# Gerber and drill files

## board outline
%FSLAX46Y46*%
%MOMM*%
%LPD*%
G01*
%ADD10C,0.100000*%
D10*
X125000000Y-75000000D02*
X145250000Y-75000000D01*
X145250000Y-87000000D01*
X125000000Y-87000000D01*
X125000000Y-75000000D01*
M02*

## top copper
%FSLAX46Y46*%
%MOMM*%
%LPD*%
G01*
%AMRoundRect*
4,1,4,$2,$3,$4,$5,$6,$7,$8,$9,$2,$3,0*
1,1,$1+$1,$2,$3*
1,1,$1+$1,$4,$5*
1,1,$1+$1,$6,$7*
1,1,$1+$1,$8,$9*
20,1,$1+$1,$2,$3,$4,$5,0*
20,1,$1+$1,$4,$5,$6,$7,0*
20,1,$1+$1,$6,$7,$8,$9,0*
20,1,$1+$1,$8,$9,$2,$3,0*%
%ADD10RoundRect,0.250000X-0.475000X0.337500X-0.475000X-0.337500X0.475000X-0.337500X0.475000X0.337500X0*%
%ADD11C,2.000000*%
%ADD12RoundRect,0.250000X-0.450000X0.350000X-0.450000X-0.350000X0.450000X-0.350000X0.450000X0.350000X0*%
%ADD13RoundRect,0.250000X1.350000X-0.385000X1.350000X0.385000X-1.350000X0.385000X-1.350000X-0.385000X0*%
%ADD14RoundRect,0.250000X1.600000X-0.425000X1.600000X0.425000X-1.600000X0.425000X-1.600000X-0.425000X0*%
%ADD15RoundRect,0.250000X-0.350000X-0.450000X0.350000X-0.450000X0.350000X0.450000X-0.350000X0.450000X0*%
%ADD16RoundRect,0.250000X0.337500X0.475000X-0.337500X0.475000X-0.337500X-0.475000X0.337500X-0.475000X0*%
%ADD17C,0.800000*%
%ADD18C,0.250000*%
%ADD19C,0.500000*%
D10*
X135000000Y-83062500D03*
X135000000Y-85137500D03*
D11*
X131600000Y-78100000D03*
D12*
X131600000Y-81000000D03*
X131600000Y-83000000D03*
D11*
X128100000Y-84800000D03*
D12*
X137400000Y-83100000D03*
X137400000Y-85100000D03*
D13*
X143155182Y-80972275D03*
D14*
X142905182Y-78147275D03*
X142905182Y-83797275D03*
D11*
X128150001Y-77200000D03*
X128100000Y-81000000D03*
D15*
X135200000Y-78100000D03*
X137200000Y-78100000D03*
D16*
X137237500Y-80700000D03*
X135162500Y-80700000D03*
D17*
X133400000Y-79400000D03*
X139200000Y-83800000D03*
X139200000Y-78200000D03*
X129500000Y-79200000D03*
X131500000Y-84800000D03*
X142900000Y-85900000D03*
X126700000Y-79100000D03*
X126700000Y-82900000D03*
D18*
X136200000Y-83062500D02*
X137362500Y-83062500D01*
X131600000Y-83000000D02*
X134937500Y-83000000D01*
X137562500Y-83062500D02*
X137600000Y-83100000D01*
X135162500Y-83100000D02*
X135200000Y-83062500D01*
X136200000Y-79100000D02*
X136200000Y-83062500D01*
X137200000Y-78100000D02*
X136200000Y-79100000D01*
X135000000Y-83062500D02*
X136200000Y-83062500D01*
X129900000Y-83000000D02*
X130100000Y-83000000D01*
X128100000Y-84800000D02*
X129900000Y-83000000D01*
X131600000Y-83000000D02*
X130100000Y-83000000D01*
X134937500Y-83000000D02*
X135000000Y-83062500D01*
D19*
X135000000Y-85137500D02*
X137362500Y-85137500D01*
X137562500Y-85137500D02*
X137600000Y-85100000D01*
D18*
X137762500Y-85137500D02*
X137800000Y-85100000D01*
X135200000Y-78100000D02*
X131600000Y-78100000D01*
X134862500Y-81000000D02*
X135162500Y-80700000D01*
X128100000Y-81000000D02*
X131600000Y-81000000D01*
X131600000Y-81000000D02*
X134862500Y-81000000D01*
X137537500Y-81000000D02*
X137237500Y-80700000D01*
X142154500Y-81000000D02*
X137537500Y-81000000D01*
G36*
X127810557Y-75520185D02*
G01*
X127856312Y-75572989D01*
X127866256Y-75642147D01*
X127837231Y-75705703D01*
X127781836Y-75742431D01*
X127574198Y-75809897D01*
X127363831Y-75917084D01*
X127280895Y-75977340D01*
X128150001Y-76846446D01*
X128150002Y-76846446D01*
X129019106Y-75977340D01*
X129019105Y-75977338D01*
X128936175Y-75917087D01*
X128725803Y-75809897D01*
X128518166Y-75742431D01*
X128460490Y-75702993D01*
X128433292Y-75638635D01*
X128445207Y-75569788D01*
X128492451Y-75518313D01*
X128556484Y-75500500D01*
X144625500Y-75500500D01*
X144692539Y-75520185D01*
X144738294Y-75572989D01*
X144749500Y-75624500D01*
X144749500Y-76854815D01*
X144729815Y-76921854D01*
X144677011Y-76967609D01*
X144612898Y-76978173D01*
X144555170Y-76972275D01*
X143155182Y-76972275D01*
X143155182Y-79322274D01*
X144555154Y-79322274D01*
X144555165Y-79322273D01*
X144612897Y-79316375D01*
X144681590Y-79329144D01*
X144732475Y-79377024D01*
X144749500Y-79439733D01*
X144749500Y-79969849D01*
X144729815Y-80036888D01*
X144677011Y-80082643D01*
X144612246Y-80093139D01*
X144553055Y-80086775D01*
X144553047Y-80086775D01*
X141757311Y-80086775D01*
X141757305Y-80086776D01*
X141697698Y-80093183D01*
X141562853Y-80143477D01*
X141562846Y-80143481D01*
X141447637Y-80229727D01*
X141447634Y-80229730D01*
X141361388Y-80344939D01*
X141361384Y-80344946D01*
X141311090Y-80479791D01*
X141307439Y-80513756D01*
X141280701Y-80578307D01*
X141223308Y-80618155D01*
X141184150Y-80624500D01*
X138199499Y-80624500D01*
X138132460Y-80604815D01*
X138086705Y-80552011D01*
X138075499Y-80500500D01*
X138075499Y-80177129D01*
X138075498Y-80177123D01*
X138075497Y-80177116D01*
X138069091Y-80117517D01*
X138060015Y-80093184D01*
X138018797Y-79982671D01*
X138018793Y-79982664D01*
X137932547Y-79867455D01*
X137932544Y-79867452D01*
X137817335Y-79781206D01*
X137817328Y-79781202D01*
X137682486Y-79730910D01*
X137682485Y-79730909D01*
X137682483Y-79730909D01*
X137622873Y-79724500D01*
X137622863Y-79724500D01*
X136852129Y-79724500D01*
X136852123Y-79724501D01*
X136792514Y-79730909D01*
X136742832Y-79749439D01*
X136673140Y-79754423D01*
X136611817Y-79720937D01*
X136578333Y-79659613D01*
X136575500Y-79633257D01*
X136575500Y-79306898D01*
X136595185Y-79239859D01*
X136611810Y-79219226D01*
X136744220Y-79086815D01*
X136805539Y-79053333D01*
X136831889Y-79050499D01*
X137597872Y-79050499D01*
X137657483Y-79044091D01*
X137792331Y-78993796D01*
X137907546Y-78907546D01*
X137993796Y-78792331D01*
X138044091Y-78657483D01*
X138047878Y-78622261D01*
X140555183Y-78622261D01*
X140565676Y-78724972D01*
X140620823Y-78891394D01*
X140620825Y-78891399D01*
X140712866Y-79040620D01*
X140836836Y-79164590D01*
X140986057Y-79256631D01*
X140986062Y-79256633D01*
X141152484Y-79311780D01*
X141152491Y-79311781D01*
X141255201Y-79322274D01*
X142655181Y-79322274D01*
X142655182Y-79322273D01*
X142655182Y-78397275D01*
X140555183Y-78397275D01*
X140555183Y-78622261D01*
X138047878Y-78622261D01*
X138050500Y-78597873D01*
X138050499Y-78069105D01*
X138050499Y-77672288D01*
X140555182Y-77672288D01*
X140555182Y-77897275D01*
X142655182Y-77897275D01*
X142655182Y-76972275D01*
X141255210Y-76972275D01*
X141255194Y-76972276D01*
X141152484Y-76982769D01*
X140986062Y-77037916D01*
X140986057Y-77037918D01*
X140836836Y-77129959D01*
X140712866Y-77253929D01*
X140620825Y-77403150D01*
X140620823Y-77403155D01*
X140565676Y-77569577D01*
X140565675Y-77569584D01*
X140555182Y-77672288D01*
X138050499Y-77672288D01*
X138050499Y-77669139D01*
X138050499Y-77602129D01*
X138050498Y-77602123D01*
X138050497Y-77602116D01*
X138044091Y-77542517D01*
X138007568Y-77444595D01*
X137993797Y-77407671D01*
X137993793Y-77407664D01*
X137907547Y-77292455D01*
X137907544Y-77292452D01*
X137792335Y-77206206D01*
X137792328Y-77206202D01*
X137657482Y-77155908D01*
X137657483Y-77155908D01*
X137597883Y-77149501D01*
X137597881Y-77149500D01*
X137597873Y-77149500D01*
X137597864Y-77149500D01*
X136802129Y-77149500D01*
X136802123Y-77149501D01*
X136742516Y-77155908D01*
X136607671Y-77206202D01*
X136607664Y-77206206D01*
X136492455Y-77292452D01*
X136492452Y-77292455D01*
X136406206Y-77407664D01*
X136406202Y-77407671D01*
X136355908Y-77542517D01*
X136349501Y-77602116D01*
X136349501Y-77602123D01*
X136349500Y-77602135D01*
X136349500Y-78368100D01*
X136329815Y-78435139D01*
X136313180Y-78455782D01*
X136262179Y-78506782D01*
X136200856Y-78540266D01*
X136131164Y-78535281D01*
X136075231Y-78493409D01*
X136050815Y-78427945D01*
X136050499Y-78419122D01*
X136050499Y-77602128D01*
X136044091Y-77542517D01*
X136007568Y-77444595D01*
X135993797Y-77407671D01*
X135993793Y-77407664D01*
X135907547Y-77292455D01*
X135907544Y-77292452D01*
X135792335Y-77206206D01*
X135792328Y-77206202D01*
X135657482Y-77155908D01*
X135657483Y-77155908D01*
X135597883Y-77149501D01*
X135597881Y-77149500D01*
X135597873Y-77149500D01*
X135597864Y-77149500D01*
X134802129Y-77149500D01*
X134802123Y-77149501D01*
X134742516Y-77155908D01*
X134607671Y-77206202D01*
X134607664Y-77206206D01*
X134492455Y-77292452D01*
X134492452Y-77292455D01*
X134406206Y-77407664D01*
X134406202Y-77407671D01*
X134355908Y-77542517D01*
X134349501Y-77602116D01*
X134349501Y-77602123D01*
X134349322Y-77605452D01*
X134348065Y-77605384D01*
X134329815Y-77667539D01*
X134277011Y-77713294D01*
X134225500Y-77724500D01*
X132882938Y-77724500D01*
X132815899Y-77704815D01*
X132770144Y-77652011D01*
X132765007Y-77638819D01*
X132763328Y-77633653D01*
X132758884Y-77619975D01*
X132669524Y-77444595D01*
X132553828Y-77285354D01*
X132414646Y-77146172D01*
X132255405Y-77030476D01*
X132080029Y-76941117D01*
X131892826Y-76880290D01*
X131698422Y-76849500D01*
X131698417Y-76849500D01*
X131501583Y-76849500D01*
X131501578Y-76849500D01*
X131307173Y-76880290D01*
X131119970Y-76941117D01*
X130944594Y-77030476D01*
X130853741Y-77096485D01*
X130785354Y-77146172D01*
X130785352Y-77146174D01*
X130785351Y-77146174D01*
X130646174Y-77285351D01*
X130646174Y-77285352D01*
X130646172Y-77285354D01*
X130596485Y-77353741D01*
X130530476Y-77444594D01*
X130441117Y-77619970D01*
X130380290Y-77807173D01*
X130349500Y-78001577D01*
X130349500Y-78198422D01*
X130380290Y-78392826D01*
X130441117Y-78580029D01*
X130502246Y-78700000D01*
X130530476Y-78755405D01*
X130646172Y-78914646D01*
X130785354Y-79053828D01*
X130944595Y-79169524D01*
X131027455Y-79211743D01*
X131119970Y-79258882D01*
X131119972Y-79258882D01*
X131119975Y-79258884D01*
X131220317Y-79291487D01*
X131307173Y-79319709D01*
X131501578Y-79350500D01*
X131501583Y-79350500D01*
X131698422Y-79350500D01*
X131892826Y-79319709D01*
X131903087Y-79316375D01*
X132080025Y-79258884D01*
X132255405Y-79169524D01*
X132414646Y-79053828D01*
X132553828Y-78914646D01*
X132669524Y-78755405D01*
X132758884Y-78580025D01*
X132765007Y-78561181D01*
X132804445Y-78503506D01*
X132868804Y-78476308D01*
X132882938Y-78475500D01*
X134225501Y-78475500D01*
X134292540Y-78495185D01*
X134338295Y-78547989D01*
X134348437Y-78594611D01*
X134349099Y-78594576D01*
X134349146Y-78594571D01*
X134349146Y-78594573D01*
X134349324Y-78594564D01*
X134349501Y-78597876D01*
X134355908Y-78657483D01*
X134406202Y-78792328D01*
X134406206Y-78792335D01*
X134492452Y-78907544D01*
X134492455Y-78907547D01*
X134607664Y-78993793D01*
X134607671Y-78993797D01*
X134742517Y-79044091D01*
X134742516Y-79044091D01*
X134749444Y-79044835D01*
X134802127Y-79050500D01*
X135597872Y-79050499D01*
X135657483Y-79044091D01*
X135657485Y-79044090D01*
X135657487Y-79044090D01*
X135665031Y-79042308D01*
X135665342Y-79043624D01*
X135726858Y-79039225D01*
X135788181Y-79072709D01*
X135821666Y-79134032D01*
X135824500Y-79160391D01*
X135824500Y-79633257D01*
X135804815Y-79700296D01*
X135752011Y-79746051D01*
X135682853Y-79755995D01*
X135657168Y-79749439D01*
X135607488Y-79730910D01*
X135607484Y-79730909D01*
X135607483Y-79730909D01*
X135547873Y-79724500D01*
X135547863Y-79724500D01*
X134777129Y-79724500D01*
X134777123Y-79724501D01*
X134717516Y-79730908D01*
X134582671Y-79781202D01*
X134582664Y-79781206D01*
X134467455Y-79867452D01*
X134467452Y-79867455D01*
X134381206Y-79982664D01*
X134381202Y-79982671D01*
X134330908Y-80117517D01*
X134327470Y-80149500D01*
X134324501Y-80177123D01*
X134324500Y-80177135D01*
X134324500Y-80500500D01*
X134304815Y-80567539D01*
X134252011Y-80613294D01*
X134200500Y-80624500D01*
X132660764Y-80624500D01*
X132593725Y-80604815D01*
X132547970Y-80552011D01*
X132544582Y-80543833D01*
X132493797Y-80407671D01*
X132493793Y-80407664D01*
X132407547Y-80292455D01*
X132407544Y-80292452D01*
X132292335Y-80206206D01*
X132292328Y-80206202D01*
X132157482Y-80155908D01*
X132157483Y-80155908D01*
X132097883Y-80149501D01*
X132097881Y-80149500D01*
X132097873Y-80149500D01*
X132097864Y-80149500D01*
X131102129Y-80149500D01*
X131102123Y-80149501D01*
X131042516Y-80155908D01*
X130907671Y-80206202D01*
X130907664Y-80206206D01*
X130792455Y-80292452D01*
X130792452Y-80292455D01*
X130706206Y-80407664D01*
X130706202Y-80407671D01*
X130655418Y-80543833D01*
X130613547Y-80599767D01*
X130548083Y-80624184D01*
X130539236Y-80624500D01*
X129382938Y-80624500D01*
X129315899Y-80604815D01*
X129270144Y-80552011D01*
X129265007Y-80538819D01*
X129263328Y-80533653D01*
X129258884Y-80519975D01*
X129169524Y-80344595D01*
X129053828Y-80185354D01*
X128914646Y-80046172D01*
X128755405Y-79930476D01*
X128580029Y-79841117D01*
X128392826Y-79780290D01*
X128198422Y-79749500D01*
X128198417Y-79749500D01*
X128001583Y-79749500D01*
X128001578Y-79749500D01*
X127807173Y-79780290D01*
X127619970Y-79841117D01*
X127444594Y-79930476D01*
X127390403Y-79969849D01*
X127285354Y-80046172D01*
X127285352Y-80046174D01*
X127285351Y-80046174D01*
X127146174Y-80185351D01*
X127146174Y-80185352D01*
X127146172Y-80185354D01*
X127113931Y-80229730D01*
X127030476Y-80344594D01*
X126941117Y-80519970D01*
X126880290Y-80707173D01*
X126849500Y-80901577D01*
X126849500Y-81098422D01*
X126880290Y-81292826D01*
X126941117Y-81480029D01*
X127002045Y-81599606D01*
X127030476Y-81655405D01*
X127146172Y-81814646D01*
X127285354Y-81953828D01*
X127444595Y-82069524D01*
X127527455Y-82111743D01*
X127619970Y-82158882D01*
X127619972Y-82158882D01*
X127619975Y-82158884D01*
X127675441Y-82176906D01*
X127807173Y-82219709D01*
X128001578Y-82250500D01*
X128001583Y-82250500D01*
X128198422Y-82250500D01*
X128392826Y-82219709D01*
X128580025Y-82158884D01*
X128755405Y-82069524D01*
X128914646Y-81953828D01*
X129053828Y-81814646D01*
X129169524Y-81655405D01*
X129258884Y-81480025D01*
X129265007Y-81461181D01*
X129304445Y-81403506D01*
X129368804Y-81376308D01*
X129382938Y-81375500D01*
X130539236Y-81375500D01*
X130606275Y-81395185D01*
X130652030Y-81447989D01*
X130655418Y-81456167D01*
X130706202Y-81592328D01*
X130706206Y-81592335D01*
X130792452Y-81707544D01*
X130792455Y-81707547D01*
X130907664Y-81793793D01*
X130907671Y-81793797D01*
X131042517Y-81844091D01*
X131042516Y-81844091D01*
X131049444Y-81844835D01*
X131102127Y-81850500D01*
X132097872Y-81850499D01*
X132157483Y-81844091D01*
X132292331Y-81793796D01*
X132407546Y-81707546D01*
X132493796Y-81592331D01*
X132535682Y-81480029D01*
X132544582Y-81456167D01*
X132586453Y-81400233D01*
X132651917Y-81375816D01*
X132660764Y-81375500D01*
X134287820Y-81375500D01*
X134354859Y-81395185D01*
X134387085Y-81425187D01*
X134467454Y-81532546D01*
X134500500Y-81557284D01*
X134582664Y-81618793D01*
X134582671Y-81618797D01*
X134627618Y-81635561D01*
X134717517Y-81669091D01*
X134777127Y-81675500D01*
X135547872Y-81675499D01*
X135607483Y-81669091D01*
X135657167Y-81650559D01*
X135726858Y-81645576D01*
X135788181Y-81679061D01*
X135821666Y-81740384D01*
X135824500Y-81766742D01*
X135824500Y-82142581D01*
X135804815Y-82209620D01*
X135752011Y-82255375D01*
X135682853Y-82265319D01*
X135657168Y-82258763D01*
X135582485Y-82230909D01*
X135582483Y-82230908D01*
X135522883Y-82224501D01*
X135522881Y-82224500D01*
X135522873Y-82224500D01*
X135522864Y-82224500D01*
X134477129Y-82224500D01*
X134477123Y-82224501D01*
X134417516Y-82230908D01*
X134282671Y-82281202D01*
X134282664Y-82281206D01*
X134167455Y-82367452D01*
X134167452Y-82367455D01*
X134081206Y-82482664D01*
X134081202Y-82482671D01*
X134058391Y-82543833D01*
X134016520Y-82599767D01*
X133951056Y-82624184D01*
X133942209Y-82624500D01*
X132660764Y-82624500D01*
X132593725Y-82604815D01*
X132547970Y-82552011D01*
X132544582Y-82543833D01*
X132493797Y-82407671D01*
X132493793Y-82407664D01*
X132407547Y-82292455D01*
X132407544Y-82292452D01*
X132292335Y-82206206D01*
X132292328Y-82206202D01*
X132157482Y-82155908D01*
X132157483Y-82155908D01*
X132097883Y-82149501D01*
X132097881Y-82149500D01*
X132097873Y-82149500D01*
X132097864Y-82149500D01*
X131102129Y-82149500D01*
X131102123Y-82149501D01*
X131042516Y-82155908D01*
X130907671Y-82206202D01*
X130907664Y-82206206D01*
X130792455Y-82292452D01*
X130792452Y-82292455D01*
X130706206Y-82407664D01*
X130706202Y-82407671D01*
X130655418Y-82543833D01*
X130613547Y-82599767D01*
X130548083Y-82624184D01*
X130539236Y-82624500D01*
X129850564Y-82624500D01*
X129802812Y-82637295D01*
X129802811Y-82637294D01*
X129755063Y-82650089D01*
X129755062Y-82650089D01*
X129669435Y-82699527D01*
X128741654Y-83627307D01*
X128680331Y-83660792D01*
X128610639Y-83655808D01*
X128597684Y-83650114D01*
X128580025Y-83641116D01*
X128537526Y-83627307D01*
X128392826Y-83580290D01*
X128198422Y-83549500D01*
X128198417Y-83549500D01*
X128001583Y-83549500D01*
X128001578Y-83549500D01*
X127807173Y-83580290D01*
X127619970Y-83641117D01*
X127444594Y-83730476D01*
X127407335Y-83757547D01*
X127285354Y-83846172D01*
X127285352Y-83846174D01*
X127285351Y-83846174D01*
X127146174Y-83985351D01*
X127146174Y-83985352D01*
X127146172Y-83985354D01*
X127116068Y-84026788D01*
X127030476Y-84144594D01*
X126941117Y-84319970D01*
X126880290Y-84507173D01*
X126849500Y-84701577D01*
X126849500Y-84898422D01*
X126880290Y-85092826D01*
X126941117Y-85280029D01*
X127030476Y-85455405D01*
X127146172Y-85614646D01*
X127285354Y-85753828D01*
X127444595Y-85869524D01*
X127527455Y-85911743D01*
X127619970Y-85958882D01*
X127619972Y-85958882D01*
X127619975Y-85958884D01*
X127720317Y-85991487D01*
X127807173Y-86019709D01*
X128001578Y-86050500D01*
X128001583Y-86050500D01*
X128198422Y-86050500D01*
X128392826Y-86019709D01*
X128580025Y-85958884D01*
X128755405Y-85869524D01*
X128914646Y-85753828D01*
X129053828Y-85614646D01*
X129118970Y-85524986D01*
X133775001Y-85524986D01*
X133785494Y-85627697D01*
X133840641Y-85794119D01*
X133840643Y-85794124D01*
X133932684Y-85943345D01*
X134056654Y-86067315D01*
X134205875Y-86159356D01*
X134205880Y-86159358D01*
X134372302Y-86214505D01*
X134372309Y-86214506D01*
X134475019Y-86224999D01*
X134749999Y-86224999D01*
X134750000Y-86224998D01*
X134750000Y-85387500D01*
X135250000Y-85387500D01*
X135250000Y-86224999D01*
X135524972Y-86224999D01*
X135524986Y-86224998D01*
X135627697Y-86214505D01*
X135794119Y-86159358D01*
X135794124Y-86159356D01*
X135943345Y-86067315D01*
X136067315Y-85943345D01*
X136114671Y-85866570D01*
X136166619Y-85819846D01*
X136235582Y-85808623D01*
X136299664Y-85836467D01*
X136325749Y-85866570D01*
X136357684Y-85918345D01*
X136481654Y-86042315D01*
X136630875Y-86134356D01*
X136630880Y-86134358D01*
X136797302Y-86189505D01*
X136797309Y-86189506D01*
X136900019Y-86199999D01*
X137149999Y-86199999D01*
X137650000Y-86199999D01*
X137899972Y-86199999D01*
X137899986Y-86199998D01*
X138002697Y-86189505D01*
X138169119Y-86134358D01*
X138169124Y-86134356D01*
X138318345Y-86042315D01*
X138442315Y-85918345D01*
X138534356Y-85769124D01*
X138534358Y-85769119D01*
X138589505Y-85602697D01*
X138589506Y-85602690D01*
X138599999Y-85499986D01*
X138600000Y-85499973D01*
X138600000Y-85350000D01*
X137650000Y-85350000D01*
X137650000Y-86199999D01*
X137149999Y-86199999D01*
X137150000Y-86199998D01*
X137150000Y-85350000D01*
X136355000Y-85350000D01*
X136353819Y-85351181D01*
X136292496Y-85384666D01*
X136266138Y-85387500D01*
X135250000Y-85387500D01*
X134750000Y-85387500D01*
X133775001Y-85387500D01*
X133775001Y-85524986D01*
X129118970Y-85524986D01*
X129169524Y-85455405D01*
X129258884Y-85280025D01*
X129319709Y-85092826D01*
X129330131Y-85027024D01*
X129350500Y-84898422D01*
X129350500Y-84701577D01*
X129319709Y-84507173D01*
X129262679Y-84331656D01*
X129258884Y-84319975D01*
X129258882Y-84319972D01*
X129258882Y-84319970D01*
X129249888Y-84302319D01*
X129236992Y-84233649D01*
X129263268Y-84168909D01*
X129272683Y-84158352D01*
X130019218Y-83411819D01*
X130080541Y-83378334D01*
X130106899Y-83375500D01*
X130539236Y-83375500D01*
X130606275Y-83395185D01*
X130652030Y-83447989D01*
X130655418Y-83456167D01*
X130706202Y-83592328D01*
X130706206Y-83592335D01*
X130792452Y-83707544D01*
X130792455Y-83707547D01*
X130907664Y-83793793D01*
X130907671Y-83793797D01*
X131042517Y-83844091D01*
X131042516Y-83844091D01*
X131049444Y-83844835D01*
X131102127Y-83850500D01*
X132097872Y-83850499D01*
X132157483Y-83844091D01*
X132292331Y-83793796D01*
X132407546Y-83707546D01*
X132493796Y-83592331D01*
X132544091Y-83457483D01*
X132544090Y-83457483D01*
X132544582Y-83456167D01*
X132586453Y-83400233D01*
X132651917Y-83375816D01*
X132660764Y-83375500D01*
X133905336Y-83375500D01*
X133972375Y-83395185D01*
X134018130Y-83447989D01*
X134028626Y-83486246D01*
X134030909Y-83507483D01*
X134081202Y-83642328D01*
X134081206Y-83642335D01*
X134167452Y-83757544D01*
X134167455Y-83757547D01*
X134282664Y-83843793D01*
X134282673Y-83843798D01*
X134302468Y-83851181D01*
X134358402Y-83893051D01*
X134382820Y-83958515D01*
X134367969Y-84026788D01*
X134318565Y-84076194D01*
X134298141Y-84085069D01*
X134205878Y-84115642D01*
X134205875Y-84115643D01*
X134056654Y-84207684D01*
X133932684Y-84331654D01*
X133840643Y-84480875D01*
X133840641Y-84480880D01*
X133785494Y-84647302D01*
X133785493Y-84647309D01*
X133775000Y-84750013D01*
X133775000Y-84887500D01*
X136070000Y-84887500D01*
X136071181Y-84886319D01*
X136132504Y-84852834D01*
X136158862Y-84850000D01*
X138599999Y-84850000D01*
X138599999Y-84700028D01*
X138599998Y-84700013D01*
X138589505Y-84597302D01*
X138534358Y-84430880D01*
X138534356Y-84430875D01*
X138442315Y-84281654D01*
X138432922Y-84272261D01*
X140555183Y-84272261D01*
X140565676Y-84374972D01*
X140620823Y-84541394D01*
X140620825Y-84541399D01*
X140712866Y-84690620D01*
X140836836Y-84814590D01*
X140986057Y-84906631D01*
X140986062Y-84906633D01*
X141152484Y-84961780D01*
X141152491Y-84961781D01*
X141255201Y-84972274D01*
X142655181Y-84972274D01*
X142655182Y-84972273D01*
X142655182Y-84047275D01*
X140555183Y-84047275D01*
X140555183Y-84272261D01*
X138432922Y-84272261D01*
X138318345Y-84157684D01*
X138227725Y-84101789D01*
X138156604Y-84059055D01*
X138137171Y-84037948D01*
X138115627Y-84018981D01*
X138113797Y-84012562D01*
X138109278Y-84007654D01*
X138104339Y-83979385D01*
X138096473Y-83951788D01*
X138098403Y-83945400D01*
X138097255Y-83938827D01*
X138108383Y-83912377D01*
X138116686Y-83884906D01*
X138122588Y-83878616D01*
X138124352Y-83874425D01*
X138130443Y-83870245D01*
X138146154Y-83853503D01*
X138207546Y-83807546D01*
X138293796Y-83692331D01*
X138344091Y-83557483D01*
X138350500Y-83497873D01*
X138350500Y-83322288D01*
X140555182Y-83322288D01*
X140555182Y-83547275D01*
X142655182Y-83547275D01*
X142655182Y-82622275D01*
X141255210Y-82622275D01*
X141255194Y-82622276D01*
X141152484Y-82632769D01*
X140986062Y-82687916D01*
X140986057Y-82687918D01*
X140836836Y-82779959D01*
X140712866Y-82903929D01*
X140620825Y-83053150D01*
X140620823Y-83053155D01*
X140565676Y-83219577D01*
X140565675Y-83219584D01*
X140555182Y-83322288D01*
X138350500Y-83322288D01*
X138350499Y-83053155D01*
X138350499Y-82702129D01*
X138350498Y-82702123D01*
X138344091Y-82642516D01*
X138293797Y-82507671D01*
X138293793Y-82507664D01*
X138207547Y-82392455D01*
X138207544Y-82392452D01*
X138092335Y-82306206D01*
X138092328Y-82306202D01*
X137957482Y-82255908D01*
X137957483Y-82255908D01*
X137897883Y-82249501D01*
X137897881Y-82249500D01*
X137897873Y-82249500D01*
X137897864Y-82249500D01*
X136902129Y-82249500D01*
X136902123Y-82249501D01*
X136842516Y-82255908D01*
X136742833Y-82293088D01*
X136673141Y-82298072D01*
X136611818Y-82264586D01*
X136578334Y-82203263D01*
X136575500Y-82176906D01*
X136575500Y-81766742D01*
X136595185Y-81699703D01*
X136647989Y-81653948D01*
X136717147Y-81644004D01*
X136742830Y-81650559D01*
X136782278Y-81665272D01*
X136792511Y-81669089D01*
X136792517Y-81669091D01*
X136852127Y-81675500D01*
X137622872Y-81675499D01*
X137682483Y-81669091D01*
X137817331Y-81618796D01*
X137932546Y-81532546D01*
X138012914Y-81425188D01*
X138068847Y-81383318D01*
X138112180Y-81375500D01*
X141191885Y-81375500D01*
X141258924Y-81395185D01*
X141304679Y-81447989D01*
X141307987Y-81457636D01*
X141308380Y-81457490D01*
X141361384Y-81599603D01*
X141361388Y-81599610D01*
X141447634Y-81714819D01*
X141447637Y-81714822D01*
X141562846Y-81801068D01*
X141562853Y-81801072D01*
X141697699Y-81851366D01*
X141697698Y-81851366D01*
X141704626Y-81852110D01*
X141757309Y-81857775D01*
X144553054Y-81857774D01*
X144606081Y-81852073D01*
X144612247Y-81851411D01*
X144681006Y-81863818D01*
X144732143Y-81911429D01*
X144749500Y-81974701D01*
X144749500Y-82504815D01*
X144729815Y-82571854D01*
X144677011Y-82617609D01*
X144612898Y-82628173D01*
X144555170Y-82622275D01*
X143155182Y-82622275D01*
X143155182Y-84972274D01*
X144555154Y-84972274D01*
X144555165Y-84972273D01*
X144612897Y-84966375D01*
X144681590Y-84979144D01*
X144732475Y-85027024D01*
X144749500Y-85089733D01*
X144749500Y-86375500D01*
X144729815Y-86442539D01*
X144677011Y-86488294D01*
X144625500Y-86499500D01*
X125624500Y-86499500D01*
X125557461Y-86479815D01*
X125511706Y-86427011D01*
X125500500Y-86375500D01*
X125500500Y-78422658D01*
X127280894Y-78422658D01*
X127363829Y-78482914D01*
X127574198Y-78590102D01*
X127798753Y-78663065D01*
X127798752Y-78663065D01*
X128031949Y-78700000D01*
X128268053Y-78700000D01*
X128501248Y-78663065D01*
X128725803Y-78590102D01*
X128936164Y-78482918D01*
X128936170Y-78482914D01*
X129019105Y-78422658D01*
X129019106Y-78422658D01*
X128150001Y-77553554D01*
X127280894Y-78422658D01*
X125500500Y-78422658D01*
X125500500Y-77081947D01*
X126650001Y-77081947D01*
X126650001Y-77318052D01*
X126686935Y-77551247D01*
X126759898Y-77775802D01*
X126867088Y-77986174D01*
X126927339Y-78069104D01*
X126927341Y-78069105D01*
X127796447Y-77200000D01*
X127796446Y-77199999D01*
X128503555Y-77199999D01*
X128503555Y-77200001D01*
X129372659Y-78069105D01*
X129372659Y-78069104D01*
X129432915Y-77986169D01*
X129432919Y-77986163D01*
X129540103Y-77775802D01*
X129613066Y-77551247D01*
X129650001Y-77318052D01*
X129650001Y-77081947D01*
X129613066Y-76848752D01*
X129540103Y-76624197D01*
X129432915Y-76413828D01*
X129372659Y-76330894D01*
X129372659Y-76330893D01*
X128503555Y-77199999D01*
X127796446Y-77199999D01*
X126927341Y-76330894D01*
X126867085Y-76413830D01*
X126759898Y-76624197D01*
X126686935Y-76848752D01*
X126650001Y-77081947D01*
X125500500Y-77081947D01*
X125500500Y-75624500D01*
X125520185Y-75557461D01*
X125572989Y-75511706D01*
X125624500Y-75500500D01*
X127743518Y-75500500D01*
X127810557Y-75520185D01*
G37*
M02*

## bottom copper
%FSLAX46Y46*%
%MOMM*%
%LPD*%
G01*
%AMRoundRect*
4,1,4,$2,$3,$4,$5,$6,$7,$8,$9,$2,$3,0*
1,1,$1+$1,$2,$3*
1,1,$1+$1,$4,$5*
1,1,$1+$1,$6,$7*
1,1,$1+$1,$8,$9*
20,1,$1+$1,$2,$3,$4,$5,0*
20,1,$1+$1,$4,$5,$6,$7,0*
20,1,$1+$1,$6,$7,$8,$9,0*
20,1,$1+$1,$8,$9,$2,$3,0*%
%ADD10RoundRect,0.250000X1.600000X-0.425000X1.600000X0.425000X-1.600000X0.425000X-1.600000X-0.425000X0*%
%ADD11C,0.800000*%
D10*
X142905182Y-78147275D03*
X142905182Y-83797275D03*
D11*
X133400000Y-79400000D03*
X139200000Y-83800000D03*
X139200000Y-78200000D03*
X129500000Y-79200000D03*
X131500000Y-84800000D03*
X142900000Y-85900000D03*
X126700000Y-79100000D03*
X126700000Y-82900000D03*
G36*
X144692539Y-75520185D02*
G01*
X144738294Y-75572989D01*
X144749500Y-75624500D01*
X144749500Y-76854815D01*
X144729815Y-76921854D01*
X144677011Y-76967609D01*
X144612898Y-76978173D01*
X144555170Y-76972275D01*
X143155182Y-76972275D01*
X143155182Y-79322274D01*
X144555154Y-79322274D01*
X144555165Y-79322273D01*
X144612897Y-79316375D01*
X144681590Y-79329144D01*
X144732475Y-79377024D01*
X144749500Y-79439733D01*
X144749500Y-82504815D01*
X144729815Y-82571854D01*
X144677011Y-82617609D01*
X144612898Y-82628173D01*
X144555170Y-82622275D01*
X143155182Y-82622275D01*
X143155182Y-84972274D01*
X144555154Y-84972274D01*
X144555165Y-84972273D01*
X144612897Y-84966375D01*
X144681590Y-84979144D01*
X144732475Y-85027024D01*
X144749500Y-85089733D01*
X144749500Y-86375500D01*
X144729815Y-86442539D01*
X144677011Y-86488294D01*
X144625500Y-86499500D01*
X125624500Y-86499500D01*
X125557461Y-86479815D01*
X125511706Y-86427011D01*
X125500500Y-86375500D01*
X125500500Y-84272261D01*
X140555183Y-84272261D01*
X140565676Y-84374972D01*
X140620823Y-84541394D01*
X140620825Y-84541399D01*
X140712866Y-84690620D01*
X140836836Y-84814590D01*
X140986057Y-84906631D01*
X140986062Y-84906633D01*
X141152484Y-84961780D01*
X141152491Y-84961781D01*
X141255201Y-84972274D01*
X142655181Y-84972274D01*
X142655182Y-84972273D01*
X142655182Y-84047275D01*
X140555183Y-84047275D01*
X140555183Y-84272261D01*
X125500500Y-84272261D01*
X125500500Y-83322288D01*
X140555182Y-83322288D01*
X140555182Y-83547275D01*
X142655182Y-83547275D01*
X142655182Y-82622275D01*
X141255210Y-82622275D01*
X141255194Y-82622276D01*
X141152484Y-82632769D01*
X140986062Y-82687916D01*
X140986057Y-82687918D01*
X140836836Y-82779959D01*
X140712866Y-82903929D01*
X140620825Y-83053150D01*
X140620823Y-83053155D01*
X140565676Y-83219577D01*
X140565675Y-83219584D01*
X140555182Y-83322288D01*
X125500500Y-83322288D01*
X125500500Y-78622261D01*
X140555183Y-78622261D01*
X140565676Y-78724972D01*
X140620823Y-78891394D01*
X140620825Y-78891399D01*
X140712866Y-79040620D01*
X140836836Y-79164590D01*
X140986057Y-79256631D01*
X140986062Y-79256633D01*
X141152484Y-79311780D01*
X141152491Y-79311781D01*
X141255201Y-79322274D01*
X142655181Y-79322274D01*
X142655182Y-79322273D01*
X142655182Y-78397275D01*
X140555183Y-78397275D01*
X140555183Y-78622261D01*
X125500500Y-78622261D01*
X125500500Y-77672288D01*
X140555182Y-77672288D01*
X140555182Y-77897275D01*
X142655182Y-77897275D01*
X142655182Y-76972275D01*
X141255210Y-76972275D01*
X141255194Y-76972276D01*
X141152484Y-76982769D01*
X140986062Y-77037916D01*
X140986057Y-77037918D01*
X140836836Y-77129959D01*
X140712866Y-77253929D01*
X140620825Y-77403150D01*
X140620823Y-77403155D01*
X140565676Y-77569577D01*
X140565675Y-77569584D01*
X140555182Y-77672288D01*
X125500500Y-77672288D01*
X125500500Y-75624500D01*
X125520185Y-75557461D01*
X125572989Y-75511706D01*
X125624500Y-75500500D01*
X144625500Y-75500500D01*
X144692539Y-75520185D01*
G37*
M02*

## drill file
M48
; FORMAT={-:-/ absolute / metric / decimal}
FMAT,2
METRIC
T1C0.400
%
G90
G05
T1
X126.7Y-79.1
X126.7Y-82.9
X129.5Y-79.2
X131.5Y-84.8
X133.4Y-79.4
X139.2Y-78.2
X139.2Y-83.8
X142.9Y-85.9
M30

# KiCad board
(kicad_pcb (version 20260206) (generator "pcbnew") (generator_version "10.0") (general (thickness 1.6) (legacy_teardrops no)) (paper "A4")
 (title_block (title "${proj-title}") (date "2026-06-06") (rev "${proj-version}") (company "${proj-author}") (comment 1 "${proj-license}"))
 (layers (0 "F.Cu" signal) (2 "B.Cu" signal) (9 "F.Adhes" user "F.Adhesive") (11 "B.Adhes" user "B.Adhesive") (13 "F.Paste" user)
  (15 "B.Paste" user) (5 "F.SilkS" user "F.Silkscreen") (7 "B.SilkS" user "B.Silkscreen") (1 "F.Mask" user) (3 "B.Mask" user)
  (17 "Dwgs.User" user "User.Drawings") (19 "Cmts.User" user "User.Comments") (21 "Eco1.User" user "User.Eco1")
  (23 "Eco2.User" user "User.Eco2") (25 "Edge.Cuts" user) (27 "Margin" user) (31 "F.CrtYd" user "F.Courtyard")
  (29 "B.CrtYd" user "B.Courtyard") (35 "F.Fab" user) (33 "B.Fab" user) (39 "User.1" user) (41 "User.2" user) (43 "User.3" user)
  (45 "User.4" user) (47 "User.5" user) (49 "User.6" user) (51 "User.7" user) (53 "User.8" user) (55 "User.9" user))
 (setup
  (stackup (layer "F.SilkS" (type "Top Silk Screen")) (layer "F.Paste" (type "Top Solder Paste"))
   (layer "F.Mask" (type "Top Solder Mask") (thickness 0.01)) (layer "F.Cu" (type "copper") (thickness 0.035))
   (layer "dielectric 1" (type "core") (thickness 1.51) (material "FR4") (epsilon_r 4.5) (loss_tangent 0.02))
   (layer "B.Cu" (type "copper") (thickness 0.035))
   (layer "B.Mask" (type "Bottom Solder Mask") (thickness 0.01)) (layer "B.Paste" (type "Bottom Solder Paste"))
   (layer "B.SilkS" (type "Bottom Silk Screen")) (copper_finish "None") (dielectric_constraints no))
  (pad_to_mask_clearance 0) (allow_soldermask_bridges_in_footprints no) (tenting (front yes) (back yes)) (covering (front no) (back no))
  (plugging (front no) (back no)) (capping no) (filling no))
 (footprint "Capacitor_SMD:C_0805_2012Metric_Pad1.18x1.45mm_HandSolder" (layer "F.Cu") (at 135 84.1 -90)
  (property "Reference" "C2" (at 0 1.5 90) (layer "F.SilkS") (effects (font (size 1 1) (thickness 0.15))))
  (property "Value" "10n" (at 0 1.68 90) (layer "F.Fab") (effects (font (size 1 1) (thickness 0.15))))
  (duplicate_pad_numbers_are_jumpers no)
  (pad "1" smd roundrect (at -1.0375 0 270) (size 1.175 1.45) (layers "F.Cu" "F.Mask" "F.Paste") (roundrect_rratio 0.212766) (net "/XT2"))
  (pad "2" smd roundrect (at 1.0375 0 270) (size 1.175 1.45) (layers "F.Cu" "F.Mask" "F.Paste") (roundrect_rratio 0.212766) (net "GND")))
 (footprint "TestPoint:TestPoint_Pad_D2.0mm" (layer "F.Cu") (at 131.6 78.1)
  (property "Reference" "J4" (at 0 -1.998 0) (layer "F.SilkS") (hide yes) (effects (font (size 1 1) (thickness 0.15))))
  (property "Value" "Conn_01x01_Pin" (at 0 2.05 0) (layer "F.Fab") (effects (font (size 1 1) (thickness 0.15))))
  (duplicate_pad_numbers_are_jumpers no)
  (pad "1" smd circle (at 0 0) (size 2 2) (layers "F.Cu" "F.Mask") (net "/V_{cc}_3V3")))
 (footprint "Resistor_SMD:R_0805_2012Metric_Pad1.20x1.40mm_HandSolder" (layer "F.Cu") (at 131.6 82 -90)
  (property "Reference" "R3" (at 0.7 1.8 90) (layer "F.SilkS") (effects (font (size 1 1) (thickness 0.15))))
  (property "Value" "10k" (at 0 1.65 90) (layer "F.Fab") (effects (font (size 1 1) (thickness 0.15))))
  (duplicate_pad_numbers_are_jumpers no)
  (pad "1" smd roundrect (at -1 0 270) (size 1.2 1.4) (layers "F.Cu" "F.Mask" "F.Paste") (roundrect_rratio 0.208333) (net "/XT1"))
  (pad "2" smd roundrect (at 1 0 270) (size 1.2 1.4) (layers "F.Cu" "F.Mask" "F.Paste") (roundrect_rratio 0.208333) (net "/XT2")))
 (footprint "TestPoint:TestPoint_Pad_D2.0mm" (layer "F.Cu") (at 128.1 84.8)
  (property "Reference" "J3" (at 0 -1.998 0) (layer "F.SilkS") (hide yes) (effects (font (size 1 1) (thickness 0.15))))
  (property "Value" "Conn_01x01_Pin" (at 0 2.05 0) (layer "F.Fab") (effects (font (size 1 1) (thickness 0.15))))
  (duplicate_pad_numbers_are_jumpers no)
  (pad "1" smd circle (at 0 0) (size 2 2) (layers "F.Cu" "F.Mask") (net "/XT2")))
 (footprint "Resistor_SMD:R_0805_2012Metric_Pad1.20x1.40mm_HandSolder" (layer "F.Cu") (at 137.4 84.1 -90)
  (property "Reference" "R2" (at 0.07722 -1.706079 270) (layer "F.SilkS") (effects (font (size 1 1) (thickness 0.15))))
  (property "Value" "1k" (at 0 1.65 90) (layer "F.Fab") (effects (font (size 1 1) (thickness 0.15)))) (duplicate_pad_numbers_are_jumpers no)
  (pad "1" smd roundrect (at -1 0 270) (size 1.2 1.4) (layers "F.Cu" "F.Mask" "F.Paste") (roundrect_rratio 0.208333) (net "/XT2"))
  (pad "2" smd roundrect (at 1 0 270) (size 1.2 1.4) (layers "F.Cu" "F.Mask" "F.Paste") (roundrect_rratio 0.208333) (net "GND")))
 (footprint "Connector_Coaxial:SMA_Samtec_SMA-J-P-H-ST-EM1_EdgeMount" (layer "F.Cu") (at 143.155182 80.972275)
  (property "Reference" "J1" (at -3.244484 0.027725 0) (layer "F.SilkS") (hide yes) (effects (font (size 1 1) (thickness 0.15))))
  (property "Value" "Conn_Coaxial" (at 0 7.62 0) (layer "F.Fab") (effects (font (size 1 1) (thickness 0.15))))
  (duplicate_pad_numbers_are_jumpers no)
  (pad "1" smd roundrect (at 0 0 90) (size 1.27 3.2) (layers "F.Cu" "F.Mask") (roundrect_rratio 0.1968503937) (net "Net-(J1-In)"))
  (pad "2" smd roundrect (at -0.25 -2.825 90) (size 1.35 3.7) (layers "F.Cu" "F.Mask") (roundrect_rratio 0.1851851852) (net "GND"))
  (pad "2" smd roundrect (at -0.25 -2.825 90) (size 1.35 3.7) (layers "B.Cu" "B.Mask") (roundrect_rratio 0.1851851852) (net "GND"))
  (pad "2" smd roundrect (at -0.25 2.825 90) (size 1.35 3.7) (layers "F.Cu" "F.Mask") (roundrect_rratio 0.1851851852) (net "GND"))
  (pad "2" smd roundrect (at -0.25 2.825 90) (size 1.35 3.7) (layers "B.Cu" "B.Mask") (roundrect_rratio 0.1851851852) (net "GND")))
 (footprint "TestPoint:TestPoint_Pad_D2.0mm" (layer "F.Cu") (at 128.150001 77.2)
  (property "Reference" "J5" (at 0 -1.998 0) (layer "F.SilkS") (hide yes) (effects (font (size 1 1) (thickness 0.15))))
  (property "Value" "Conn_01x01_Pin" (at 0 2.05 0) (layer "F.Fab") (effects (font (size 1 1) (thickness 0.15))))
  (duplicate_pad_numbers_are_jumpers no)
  (pad "1" smd circle (at 0 0) (size 2 2) (layers "F.Cu" "F.Mask") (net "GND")))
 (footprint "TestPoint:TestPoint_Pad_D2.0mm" (layer "F.Cu") (at 128.1 81)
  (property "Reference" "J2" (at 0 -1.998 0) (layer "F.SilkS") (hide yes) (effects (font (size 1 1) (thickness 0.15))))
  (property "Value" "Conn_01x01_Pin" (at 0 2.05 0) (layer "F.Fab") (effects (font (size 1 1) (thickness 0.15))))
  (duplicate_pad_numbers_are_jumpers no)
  (pad "1" smd circle (at 0 0) (size 2 2) (layers "F.Cu" "F.Mask") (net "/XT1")))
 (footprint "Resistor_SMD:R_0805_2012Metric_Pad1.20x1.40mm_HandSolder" (layer "F.Cu") (at 136.2 78.1)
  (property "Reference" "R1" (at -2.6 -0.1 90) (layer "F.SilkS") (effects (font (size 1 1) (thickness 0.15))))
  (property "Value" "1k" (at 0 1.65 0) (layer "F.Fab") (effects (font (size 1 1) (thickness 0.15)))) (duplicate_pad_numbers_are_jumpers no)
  (pad "1" smd roundrect (at -1 0) (size 1.2 1.4) (layers "F.Cu" "F.Mask" "F.Paste") (roundrect_rratio 0.208333) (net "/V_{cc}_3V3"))
  (pad "2" smd roundrect (at 1 0) (size 1.2 1.4) (layers "F.Cu" "F.Mask" "F.Paste") (roundrect_rratio 0.208333) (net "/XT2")))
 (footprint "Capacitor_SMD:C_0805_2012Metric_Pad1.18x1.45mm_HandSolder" (layer "F.Cu") (at 136.2 80.7 180)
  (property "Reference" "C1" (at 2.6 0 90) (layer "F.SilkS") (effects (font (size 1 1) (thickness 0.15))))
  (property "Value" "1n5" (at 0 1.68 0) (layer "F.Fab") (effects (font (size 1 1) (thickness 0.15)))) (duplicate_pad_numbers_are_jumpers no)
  (pad "1" smd roundrect (at -1.0375 0 180) (size 1.175 1.45) (layers "F.Cu" "F.Mask" "F.Paste") (roundrect_rratio 0.212766)
   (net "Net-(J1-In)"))
  (pad "2" smd roundrect (at 1.0375 0 180) (size 1.175 1.45) (layers "F.Cu" "F.Mask" "F.Paste") (roundrect_rratio 0.212766) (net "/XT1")))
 (gr_rect (start 125 75) (end 145.25 87) (stroke (width 0.1) (type default)) (fill no) (layer "Edge.Cuts"))
 (segment (start 136.2 83.0625) (end 137.3625 83.0625) (width 0.25) (layer "F.Cu") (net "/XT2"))
 (segment (start 131.6 83) (end 134.9375 83) (width 0.25) (layer "F.Cu") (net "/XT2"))
 (segment (start 137.5625 83.0625) (end 137.6 83.1) (width 0.25) (layer "F.Cu") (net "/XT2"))
 (segment (start 135.1625 83.1) (end 135.2 83.0625) (width 0.25) (layer "F.Cu") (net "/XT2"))
 (segment (start 136.2 79.1) (end 136.2 83.0625) (width 0.25) (layer "F.Cu") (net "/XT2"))
 (segment (start 137.2 78.1) (end 136.2 79.1) (width 0.25) (layer "F.Cu") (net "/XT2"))
 (segment (start 135 83.0625) (end 136.2 83.0625) (width 0.25) (layer "F.Cu") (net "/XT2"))
 (segment (start 129.9 83) (end 130.1 83) (width 0.25) (layer "F.Cu") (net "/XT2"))
 (segment (start 128.1 84.8) (end 129.9 83) (width 0.25) (layer "F.Cu") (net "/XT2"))
 (segment (start 131.6 83) (end 130.1 83) (width 0.25) (layer "F.Cu") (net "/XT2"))
 (segment (start 134.9375 83) (end 135 83.0625) (width 0.25) (layer "F.Cu") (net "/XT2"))
 (segment (start 135 85.1375) (end 137.3625 85.1375) (width 0.5) (layer "F.Cu") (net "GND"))
 (segment (start 137.5625 85.1375) (end 137.6 85.1) (width 0.5) (layer "F.Cu") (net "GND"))
 (segment (start 137.7625 85.1375) (end 137.8 85.1) (width 0.25) (layer "F.Cu") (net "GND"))
 (via (at 133.4 79.4) (size 0.8) (drill 0.4) (layers "F.Cu" "B.Cu") (free yes) (capping no) (covering (front no) (back no))
  (plugging (front no) (back no)) (filling no) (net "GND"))
 (via (at 139.2 83.8) (size 0.8) (drill 0.4) (layers "F.Cu" "B.Cu") (free yes) (capping no) (covering (front no) (back no))
  (plugging (front no) (back no)) (filling no) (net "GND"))
 (via (at 139.2 78.2) (size 0.8) (drill 0.4) (layers "F.Cu" "B.Cu") (free yes) (capping no) (covering (front no) (back no))
  (plugging (front no) (back no)) (filling no) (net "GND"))
 (via (at 129.5 79.2) (size 0.8) (drill 0.4) (layers "F.Cu" "B.Cu") (free yes) (capping no) (covering (front no) (back no))
  (plugging (front no) (back no)) (filling no) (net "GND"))
 (via (at 131.5 84.8) (size 0.8) (drill 0.4) (layers "F.Cu" "B.Cu") (free yes) (capping no) (covering (front no) (back no))
  (plugging (front no) (back no)) (filling no) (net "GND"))
 (via (at 142.9 85.9) (size 0.8) (drill 0.4) (layers "F.Cu" "B.Cu") (free yes) (capping no) (covering (front no) (back no))
  (plugging (front no) (back no)) (filling no) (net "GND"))
 (via (at 126.7 79.1) (size 0.8) (drill 0.4) (layers "F.Cu" "B.Cu") (free yes) (capping no) (covering (front no) (back no))
  (plugging (front no) (back no)) (filling no) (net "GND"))
 (via (at 126.7 82.9) (size 0.8) (drill 0.4) (layers "F.Cu" "B.Cu") (free yes) (capping no) (covering (front no) (back no))
  (plugging (front no) (back no)) (filling no) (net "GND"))
 (segment (start 135.2 78.1) (end 131.6 78.1) (width 0.25) (layer "F.Cu") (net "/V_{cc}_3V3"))
 (segment (start 134.8625 81) (end 135.1625 80.7) (width 0.25) (layer "F.Cu") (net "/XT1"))
 (segment (start 128.1 81) (end 131.6 81) (width 0.25) (layer "F.Cu") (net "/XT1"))
 (segment (start 131.6 81) (end 134.8625 81) (width 0.25) (layer "F.Cu") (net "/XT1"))
 (segment (start 137.5375 81) (end 137.2375 80.7) (width 0.25) (layer "F.Cu") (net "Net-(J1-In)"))
 (segment (start 142.1545 81) (end 137.5375 81) (width 0.25) (layer "F.Cu") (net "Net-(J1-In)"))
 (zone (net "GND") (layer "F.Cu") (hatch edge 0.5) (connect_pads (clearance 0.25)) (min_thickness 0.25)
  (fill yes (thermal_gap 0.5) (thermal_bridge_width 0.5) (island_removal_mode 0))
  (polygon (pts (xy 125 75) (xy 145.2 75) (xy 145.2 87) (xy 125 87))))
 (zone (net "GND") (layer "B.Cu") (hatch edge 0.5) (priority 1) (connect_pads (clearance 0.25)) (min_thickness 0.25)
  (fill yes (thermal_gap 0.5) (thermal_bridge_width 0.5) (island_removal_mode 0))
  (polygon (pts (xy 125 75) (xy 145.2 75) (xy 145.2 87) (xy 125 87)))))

